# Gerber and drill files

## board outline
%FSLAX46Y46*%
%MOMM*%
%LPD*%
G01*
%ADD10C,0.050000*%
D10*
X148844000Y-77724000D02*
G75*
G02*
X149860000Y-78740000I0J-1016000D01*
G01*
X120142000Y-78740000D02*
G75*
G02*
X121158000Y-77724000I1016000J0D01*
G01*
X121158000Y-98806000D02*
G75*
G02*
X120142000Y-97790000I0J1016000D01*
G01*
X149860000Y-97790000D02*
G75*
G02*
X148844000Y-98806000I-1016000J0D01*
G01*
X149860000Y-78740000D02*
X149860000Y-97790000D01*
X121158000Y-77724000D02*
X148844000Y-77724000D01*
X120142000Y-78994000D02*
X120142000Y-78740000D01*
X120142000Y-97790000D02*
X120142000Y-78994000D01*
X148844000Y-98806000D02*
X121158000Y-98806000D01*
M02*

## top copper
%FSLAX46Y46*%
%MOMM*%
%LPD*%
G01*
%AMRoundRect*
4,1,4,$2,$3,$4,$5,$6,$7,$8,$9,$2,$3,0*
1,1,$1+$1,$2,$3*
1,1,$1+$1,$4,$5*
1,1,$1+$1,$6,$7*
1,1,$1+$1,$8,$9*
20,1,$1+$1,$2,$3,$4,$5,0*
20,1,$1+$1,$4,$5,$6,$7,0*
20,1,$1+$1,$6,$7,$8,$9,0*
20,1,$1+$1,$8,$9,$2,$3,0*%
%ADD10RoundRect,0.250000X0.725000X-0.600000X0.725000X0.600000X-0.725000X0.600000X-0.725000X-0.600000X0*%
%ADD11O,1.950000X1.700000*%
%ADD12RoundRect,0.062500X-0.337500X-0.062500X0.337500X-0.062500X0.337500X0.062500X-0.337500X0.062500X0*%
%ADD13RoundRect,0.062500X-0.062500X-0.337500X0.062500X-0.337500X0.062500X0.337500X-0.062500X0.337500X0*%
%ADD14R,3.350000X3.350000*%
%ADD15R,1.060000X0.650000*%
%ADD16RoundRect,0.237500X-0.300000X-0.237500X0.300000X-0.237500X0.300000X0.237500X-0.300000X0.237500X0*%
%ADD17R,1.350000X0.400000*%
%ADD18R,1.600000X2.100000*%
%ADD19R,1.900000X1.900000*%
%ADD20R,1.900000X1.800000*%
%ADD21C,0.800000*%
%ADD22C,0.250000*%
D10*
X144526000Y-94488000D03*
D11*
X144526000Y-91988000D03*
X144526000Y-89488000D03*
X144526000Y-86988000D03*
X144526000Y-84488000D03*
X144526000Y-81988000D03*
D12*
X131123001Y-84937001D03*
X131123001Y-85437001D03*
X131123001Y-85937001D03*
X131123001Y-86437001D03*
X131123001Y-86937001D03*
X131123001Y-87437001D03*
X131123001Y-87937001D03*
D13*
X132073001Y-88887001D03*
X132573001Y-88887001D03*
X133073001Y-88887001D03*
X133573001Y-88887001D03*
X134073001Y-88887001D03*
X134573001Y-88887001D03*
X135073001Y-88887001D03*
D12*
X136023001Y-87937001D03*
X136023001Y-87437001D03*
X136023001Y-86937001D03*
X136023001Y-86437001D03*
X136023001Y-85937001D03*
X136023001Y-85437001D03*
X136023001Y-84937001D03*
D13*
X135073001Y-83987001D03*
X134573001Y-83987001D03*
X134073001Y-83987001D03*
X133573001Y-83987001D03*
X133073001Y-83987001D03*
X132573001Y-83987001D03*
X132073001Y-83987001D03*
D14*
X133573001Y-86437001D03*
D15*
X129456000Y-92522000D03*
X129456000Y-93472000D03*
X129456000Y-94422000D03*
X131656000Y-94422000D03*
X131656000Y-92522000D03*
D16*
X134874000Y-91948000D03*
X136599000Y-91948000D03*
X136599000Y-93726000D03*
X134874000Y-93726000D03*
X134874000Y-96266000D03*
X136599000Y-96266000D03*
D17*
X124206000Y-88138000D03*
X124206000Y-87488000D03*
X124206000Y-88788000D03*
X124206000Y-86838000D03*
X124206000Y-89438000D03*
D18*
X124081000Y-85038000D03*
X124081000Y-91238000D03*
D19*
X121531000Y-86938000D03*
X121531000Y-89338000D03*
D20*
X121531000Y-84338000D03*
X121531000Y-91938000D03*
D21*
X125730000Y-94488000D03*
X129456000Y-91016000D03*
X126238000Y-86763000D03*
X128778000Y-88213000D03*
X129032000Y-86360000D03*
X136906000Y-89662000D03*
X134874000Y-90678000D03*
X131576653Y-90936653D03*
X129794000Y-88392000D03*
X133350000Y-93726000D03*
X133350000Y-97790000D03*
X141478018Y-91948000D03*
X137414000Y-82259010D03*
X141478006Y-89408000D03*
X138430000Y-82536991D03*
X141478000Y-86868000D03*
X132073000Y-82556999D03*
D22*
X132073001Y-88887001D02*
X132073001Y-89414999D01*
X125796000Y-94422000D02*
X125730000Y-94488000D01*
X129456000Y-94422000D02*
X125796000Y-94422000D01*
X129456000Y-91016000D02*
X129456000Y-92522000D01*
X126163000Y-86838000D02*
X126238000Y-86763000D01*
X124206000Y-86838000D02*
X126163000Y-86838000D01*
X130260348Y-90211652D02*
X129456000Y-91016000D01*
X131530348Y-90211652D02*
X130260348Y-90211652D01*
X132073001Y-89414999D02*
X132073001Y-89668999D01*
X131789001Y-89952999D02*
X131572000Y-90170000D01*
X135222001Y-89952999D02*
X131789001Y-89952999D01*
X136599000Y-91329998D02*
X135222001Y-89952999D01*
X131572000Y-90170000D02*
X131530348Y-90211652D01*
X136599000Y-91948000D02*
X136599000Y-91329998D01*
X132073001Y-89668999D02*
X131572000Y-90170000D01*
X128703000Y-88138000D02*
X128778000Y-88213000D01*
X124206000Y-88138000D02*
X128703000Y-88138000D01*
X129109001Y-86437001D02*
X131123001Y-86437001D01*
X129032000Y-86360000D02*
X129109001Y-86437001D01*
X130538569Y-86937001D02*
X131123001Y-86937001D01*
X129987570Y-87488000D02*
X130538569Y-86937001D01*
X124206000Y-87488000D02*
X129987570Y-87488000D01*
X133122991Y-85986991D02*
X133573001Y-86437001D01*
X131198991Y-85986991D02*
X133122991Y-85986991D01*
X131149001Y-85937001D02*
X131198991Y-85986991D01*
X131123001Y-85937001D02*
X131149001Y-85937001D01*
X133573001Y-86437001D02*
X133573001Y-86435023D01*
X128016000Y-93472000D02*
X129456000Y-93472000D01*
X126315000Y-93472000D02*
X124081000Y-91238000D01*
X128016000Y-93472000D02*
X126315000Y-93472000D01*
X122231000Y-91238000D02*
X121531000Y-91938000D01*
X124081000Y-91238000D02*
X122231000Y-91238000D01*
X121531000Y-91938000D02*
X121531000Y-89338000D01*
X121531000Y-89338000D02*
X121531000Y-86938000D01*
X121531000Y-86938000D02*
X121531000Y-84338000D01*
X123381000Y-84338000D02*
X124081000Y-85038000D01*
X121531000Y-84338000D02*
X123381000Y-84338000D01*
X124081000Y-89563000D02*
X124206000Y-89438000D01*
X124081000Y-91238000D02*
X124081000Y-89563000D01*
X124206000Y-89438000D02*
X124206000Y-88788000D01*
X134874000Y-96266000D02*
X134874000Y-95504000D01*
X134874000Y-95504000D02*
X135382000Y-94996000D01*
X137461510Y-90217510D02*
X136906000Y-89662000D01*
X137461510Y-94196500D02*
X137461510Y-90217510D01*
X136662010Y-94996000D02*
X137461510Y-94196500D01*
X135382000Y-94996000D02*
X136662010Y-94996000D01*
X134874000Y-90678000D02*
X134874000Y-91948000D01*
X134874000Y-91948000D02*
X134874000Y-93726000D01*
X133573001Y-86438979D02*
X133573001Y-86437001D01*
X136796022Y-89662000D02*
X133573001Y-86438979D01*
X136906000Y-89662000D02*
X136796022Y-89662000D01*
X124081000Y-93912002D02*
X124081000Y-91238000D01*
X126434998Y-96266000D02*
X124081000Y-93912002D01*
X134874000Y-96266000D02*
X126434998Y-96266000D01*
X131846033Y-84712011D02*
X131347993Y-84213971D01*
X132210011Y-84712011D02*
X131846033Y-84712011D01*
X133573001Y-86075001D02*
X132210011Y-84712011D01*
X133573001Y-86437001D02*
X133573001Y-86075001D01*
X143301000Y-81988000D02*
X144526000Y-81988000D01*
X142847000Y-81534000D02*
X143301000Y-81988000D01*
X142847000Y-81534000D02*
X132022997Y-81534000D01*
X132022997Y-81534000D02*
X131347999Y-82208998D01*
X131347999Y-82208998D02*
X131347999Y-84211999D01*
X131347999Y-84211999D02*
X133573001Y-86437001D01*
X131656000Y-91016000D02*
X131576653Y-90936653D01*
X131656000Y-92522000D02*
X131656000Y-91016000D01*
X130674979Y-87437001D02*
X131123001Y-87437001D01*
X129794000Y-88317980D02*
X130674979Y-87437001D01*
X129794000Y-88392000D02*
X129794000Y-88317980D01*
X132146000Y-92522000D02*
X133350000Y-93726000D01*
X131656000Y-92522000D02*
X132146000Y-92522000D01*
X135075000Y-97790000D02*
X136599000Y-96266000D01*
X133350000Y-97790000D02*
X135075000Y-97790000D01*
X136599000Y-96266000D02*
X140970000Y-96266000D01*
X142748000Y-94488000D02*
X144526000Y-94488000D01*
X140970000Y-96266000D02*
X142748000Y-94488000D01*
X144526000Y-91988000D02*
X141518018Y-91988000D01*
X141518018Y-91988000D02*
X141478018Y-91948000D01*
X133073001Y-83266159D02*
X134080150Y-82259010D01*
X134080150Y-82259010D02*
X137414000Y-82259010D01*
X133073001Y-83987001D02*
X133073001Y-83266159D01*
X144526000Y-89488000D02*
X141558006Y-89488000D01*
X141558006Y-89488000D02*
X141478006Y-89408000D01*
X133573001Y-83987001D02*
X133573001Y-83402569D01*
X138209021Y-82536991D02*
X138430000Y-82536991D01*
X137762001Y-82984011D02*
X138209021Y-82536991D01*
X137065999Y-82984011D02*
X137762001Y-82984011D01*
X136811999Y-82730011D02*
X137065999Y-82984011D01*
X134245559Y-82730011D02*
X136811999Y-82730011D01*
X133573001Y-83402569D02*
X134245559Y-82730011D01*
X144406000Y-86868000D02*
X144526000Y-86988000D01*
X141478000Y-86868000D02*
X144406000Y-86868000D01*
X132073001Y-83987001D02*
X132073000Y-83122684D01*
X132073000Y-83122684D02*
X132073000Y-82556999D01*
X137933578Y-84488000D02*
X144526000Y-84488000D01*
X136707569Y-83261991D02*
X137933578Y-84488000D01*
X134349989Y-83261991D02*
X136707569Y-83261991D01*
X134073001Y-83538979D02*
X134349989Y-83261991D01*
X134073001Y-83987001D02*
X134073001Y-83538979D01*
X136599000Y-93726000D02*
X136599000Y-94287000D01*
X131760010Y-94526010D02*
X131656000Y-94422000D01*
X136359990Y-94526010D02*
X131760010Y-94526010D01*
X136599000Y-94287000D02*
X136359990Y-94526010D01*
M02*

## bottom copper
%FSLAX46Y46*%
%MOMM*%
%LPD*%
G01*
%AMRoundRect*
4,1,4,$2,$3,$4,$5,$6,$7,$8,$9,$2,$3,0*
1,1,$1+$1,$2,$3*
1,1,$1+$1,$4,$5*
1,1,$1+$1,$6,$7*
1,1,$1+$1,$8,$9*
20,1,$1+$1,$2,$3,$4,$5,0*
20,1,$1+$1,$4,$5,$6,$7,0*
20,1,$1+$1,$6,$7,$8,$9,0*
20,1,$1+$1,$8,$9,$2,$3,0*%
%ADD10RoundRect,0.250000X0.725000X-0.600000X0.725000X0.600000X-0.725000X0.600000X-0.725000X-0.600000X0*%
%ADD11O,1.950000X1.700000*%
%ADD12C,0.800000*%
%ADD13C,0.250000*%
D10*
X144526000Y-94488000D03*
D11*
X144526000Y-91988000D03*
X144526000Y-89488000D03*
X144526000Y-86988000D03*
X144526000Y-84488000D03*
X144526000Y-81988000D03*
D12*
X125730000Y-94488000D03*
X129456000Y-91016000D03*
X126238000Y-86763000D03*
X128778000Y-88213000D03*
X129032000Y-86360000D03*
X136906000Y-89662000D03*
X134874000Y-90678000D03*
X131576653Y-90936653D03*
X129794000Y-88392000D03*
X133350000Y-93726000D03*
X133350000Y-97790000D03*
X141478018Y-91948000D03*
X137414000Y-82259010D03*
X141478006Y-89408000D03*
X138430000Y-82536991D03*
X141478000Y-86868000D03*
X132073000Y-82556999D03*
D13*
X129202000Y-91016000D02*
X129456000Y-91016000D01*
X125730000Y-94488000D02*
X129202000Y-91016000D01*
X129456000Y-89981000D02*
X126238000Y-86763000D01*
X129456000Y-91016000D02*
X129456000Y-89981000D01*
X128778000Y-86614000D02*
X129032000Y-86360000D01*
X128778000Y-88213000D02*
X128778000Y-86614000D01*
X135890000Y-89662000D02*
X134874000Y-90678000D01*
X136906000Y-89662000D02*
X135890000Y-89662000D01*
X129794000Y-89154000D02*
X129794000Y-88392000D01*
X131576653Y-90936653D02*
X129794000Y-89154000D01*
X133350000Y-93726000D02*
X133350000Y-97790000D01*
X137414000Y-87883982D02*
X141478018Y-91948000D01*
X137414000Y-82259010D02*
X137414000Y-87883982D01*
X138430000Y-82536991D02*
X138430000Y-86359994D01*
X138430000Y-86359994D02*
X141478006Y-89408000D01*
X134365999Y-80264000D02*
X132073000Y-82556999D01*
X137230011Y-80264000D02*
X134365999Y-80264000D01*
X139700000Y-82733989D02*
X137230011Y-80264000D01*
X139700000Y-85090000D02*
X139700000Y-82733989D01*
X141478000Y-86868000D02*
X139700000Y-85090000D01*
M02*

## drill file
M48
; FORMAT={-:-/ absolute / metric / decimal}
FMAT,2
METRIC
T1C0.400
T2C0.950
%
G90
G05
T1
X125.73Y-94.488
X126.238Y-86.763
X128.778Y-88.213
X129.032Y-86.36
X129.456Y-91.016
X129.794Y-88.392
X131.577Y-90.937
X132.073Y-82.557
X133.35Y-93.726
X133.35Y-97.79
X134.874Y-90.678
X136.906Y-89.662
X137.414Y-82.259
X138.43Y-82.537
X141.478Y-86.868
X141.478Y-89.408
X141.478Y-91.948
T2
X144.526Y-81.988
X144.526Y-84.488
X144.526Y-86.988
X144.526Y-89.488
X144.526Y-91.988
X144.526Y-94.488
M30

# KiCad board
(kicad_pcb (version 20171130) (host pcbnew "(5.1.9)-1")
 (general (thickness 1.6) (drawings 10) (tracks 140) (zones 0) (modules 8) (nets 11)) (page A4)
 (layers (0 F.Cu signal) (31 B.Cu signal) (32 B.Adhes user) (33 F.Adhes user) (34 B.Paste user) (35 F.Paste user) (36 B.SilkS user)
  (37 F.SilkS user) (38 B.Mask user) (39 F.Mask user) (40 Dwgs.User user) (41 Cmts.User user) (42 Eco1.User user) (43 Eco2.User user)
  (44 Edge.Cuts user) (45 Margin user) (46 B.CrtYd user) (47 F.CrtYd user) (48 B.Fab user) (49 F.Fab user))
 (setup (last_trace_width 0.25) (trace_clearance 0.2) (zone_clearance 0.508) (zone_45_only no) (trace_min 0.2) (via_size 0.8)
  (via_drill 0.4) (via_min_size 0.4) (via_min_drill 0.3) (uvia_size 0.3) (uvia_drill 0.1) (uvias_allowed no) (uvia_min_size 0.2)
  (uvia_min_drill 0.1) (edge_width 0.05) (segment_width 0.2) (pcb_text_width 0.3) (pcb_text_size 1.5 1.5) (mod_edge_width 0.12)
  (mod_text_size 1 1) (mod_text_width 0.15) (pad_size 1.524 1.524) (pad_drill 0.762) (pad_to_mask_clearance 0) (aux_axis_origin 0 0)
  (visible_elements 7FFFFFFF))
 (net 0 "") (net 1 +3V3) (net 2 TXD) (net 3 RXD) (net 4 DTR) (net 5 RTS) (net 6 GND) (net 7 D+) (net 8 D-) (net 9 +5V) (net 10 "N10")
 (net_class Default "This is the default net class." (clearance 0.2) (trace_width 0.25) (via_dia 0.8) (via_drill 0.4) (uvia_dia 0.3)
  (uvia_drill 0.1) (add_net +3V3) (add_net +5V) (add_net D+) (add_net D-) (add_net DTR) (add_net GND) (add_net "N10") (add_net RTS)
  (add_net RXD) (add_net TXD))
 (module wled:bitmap (layer F.Cu) (at 122.936 96.012)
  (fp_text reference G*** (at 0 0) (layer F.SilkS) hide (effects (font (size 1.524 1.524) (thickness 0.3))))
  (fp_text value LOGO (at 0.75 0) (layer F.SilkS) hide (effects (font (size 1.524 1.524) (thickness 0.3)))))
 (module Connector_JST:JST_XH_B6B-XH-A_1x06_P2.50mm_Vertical (layer F.Cu) (at 144.526 94.488 90)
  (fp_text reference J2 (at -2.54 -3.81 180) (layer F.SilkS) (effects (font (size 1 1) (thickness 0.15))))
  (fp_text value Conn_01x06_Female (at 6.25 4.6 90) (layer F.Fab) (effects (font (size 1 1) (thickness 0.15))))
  (pad 1 thru_hole roundrect (at 0 0 90) (size 1.7 1.95) (drill 0.95) (layers *.Cu *.Mask) (roundrect_rratio 0.1470588235294118)
   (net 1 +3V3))
  (pad 2 thru_hole oval (at 2.5 0 90) (size 1.7 1.95) (drill 0.95) (layers *.Cu *.Mask) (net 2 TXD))
  (pad 3 thru_hole oval (at 5 0 90) (size 1.7 1.95) (drill 0.95) (layers *.Cu *.Mask) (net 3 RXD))
  (pad 4 thru_hole oval (at 7.5 0 90) (size 1.7 1.95) (drill 0.95) (layers *.Cu *.Mask) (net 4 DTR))
  (pad 5 thru_hole oval (at 10 0 90) (size 1.7 1.95) (drill 0.95) (layers *.Cu *.Mask) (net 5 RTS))
  (pad 6 thru_hole oval (at 12.5 0 90) (size 1.7 1.95) (drill 0.95) (layers *.Cu *.Mask) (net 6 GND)))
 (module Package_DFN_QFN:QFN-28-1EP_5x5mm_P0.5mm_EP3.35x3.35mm (layer F.Cu) (at 133.573001 86.437001)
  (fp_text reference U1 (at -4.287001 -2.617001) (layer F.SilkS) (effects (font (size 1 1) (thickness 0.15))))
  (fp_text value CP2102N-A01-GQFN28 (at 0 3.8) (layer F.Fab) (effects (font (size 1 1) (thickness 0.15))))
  (pad 1 smd roundrect (at -2.45 -1.5) (size 0.8 0.25) (layers F.Cu F.Paste F.Mask) (roundrect_rratio 0.25))
  (pad 2 smd roundrect (at -2.45 -1) (size 0.8 0.25) (layers F.Cu F.Paste F.Mask) (roundrect_rratio 0.25))
  (pad 3 smd roundrect (at -2.45 -0.5) (size 0.8 0.25) (layers F.Cu F.Paste F.Mask) (roundrect_rratio 0.25) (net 6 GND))
  (pad 4 smd roundrect (at -2.45 0) (size 0.8 0.25) (layers F.Cu F.Paste F.Mask) (roundrect_rratio 0.25) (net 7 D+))
  (pad 5 smd roundrect (at -2.45 0.5) (size 0.8 0.25) (layers F.Cu F.Paste F.Mask) (roundrect_rratio 0.25) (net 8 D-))
  (pad 6 smd roundrect (at -2.45 1) (size 0.8 0.25) (layers F.Cu F.Paste F.Mask) (roundrect_rratio 0.25) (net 1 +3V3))
  (pad 7 smd roundrect (at -2.45 1.5) (size 0.8 0.25) (layers F.Cu F.Paste F.Mask) (roundrect_rratio 0.25))
  (pad 8 smd roundrect (at -1.5 2.45) (size 0.25 0.8) (layers F.Cu F.Paste F.Mask) (roundrect_rratio 0.25) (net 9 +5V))
  (pad 9 smd roundrect (at -1 2.45) (size 0.25 0.8) (layers F.Cu F.Paste F.Mask) (roundrect_rratio 0.25))
  (pad 10 smd roundrect (at -0.5 2.45) (size 0.25 0.8) (layers F.Cu F.Paste F.Mask) (roundrect_rratio 0.25))
  (pad 11 smd roundrect (at 0 2.45) (size 0.25 0.8) (layers F.Cu F.Paste F.Mask) (roundrect_rratio 0.25))
  (pad 12 smd roundrect (at 0.5 2.45) (size 0.25 0.8) (layers F.Cu F.Paste F.Mask) (roundrect_rratio 0.25))
  (pad 13 smd roundrect (at 1 2.45) (size 0.25 0.8) (layers F.Cu F.Paste F.Mask) (roundrect_rratio 0.25))
  (pad 14 smd roundrect (at 1.5 2.45) (size 0.25 0.8) (layers F.Cu F.Paste F.Mask) (roundrect_rratio 0.25))
  (pad 15 smd roundrect (at 2.45 1.5) (size 0.8 0.25) (layers F.Cu F.Paste F.Mask) (roundrect_rratio 0.25))
  (pad 16 smd roundrect (at 2.45 1) (size 0.8 0.25) (layers F.Cu F.Paste F.Mask) (roundrect_rratio 0.25))
  (pad 17 smd roundrect (at 2.45 0.5) (size 0.8 0.25) (layers F.Cu F.Paste F.Mask) (roundrect_rratio 0.25))
  (pad 18 smd roundrect (at 2.45 0) (size 0.8 0.25) (layers F.Cu F.Paste F.Mask) (roundrect_rratio 0.25))
  (pad 19 smd roundrect (at 2.45 -0.5) (size 0.8 0.25) (layers F.Cu F.Paste F.Mask) (roundrect_rratio 0.25))
  (pad 20 smd roundrect (at 2.45 -1) (size 0.8 0.25) (layers F.Cu F.Paste F.Mask) (roundrect_rratio 0.25))
  (pad 21 smd roundrect (at 2.45 -1.5) (size 0.8 0.25) (layers F.Cu F.Paste F.Mask) (roundrect_rratio 0.25))
  (pad 22 smd roundrect (at 1.5 -2.45) (size 0.25 0.8) (layers F.Cu F.Paste F.Mask) (roundrect_rratio 0.25))
  (pad 23 smd roundrect (at 1 -2.45) (size 0.25 0.8) (layers F.Cu F.Paste F.Mask) (roundrect_rratio 0.25))
  (pad 24 smd roundrect (at 0.5 -2.45) (size 0.25 0.8) (layers F.Cu F.Paste F.Mask) (roundrect_rratio 0.25) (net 5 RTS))
  (pad 25 smd roundrect (at 0 -2.45) (size 0.25 0.8) (layers F.Cu F.Paste F.Mask) (roundrect_rratio 0.25) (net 3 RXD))
  (pad 26 smd roundrect (at -0.5 -2.45) (size 0.25 0.8) (layers F.Cu F.Paste F.Mask) (roundrect_rratio 0.25) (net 2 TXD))
  (pad 27 smd roundrect (at -1 -2.45) (size 0.25 0.8) (layers F.Cu F.Paste F.Mask) (roundrect_rratio 0.25))
  (pad 28 smd roundrect (at -1.5 -2.45) (size 0.25 0.8) (layers F.Cu F.Paste F.Mask) (roundrect_rratio 0.25) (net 4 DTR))
  (pad 29 smd rect (at 0 0) (size 3.35 3.35) (layers F.Cu F.Mask) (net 6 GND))
  (pad "" smd roundrect (at -1.12 -1.12) (size 0.9 0.9) (layers F.Paste) (roundrect_rratio 0.25))
  (pad "" smd roundrect (at -1.12 0) (size 0.9 0.9) (layers F.Paste) (roundrect_rratio 0.25))
  (pad "" smd roundrect (at -1.12 1.12) (size 0.9 0.9) (layers F.Paste) (roundrect_rratio 0.25))
  (pad "" smd roundrect (at 0 -1.12) (size 0.9 0.9) (layers F.Paste) (roundrect_rratio 0.25))
  (pad "" smd roundrect (at 0 0) (size 0.9 0.9) (layers F.Paste) (roundrect_rratio 0.25))
  (pad "" smd roundrect (at 0 1.12) (size 0.9 0.9) (layers F.Paste) (roundrect_rratio 0.25))
  (pad "" smd roundrect (at 1.12 -1.12) (size 0.9 0.9) (layers F.Paste) (roundrect_rratio 0.25))
  (pad "" smd roundrect (at 1.12 0) (size 0.9 0.9) (layers F.Paste) (roundrect_rratio 0.25))
  (pad "" smd roundrect (at 1.12 1.12) (size 0.9 0.9) (layers F.Paste) (roundrect_rratio 0.25)))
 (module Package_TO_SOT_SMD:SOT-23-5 (layer F.Cu) (at 130.556 93.472)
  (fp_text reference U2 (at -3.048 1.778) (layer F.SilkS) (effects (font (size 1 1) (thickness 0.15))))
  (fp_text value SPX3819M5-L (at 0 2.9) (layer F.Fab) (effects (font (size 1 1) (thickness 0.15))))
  (pad 1 smd rect (at -1.1 -0.95) (size 1.06 0.65) (layers F.Cu F.Paste F.Mask) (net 9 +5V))
  (pad 2 smd rect (at -1.1 0) (size 1.06 0.65) (layers F.Cu F.Paste F.Mask) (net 6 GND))
  (pad 3 smd rect (at -1.1 0.95) (size 1.06 0.65) (layers F.Cu F.Paste F.Mask) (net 9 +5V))
  (pad 4 smd rect (at 1.1 0.95) (size 1.06 0.65) (layers F.Cu F.Paste F.Mask) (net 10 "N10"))
  (pad 5 smd rect (at 1.1 -0.95) (size 1.06 0.65) (layers F.Cu F.Paste F.Mask) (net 1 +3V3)))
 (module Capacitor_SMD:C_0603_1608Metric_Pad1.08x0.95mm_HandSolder (layer F.Cu) (at 135.7365 91.948)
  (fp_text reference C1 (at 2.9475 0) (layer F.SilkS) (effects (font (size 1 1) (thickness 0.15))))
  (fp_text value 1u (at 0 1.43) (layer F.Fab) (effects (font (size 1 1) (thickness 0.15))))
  (pad 1 smd roundrect (at -0.8625 0) (size 1.075 0.95) (layers F.Cu F.Paste F.Mask) (roundrect_rratio 0.25) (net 6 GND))
  (pad 2 smd roundrect (at 0.8625 0) (size 1.075 0.95) (layers F.Cu F.Paste F.Mask) (roundrect_rratio 0.25) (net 9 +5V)))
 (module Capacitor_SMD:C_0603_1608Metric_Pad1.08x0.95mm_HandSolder (layer F.Cu) (at 135.7365 93.726)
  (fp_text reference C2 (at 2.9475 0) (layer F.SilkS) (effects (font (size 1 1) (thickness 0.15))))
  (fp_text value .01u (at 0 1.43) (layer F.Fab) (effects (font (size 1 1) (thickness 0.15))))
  (pad 2 smd roundrect (at 0.8625 0) (size 1.075 0.95) (layers F.Cu F.Paste F.Mask) (roundrect_rratio 0.25) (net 10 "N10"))
  (pad 1 smd roundrect (at -0.8625 0) (size 1.075 0.95) (layers F.Cu F.Paste F.Mask) (roundrect_rratio 0.25) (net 6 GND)))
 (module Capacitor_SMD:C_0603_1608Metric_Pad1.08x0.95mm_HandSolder (layer F.Cu) (at 135.7365 96.266)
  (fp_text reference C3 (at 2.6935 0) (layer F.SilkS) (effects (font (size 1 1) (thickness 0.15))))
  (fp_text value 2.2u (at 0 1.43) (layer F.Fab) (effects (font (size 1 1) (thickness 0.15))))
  (pad 1 smd roundrect (at -0.8625 0) (size 1.075 0.95) (layers F.Cu F.Paste F.Mask) (roundrect_rratio 0.25) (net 6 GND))
  (pad 2 smd roundrect (at 0.8625 0) (size 1.075 0.95) (layers F.Cu F.Paste F.Mask) (roundrect_rratio 0.25) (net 1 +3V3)))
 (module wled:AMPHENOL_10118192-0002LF (layer F.Cu) (at 124.206 88.138 270)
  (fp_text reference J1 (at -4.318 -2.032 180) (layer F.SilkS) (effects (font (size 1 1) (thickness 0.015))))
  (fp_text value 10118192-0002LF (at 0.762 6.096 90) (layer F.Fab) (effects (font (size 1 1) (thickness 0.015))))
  (pad 3 smd rect (at 0 0 270) (size 0.4 1.35) (layers F.Cu F.Paste F.Mask) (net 7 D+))
  (pad 2 smd rect (at -0.65 0 270) (size 0.4 1.35) (layers F.Cu F.Paste F.Mask) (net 8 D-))
  (pad 4 smd rect (at 0.65 0 270) (size 0.4 1.35) (layers F.Cu F.Paste F.Mask) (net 6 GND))
  (pad 1 smd rect (at -1.3 0 270) (size 0.4 1.35) (layers F.Cu F.Paste F.Mask) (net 9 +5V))
  (pad 5 smd rect (at 1.3 0 270) (size 0.4 1.35) (layers F.Cu F.Paste F.Mask) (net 6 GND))
  (pad S1 smd rect (at -3.1 0.125 270) (size 2.1 1.6) (layers F.Cu F.Paste F.Mask) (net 6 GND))
  (pad S2 smd rect (at 3.1 0.125 270) (size 2.1 1.6) (layers F.Cu F.Paste F.Mask) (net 6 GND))
  (pad S4 smd rect (at -1.2 2.675 270) (size 1.9 1.9) (layers F.Cu F.Paste F.Mask) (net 6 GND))
  (pad S5 smd rect (at 1.2 2.675 270) (size 1.9 1.9) (layers F.Cu F.Paste F.Mask) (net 6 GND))
  (pad S3 smd rect (at -3.8 2.675 270) (size 1.8 1.9) (layers F.Cu F.Paste F.Mask) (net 6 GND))
  (pad S6 smd rect (at 3.8 2.675 270) (size 1.8 1.9) (layers F.Cu F.Paste F.Mask) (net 6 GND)))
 (gr_arc (start 148.844 78.74) (end 149.86 78.74) (angle -90) (layer Edge.Cuts) (width 0.05))
 (gr_arc (start 121.158 78.74) (end 121.158 77.724) (angle -90) (layer Edge.Cuts) (width 0.05))
 (gr_arc (start 121.158 97.79) (end 120.142 97.79) (angle -90) (layer Edge.Cuts) (width 0.05))
 (gr_arc (start 148.844 97.79) (end 148.844 98.806) (angle -90) (layer Edge.Cuts) (width 0.05))
 (gr_line (start 149.86 78.74) (end 149.86 97.79) (layer Edge.Cuts) (width 0.05))
 (gr_line (start 121.158 77.724) (end 148.844 77.724) (layer Edge.Cuts) (width 0.05))
 (gr_line (start 120.142 78.994) (end 120.142 78.74) (layer Edge.Cuts) (width 0.05))
 (gr_line (start 120.142 97.79) (end 120.142 78.994) (layer Edge.Cuts) (width 0.05))
 (gr_line (start 148.844 98.806) (end 121.158 98.806) (layer Edge.Cuts) (width 0.05))
 (segment (start 132.073001 88.887001) (end 132.073001 89.414999) (width 0.25) (layer F.Cu) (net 9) (status 10))
 (via (at 125.73 94.488) (size 0.8) (drill 0.4) (layers F.Cu B.Cu) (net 9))
 (segment (start 125.796 94.422) (end 125.73 94.488) (width 0.25) (layer F.Cu) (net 9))
 (segment (start 129.456 94.422) (end 125.796 94.422) (width 0.25) (layer F.Cu) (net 9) (status 10))
 (via (at 129.456 91.016) (size 0.8) (drill 0.4) (layers F.Cu B.Cu) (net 9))
 (segment (start 129.202 91.016) (end 129.456 91.016) (width 0.25) (layer B.Cu) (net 9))
 (segment (start 125.73 94.488) (end 129.202 91.016) (width 0.25) (layer B.Cu) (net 9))
 (segment (start 129.456 91.016) (end 129.456 92.522) (width 0.25) (layer F.Cu) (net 9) (status 20))
 (via (at 126.238 86.763) (size 0.8) (drill 0.4) (layers F.Cu B.Cu) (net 9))
 (segment (start 129.456 89.981) (end 126.238 86.763) (width 0.25) (layer B.Cu) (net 9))
 (segment (start 129.456 91.016) (end 129.456 89.981) (width 0.25) (layer B.Cu) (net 9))
 (segment (start 126.163 86.838) (end 126.238 86.763) (width 0.25) (layer F.Cu) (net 9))
 (segment (start 124.206 86.838) (end 126.163 86.838) (width 0.25) (layer F.Cu) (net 9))
 (segment (start 130.260348 90.211652) (end 129.456 91.016) (width 0.25) (layer F.Cu) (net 9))
 (segment (start 131.530348 90.211652) (end 130.260348 90.211652) (width 0.25) (layer F.Cu) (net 9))
 (segment (start 132.073001 89.414999) (end 132.073001 89.668999) (width 0.25) (layer F.Cu) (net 9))
 (segment (start 131.789001 89.952999) (end 131.572 90.17) (width 0.25) (layer F.Cu) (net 9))
 (segment (start 135.222001 89.952999) (end 131.789001 89.952999) (width 0.25) (layer F.Cu) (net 9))
 (segment (start 136.599 91.329998) (end 135.222001 89.952999) (width 0.25) (layer F.Cu) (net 9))
 (segment (start 131.572 90.17) (end 131.530348 90.211652) (width 0.25) (layer F.Cu) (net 9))
 (segment (start 136.599 91.948) (end 136.599 91.329998) (width 0.25) (layer F.Cu) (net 9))
 (segment (start 132.073001 89.668999) (end 131.572 90.17) (width 0.25) (layer F.Cu) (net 9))
 (via (at 128.778 88.213) (size 0.8) (drill 0.4) (layers F.Cu B.Cu) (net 7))
 (segment (start 128.703 88.138) (end 128.778 88.213) (width 0.25) (layer F.Cu) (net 7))
 (segment (start 124.206 88.138) (end 128.703 88.138) (width 0.25) (layer F.Cu) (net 7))
 (via (at 129.032 86.36) (size 0.8) (drill 0.4) (layers F.Cu B.Cu) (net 7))
 (segment (start 128.778 86.614) (end 129.032 86.36) (width 0.25) (layer B.Cu) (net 7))
 (segment (start 128.778 88.213) (end 128.778 86.614) (width 0.25) (layer B.Cu) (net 7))
 (segment (start 129.109001 86.437001) (end 131.123001 86.437001) (width 0.25) (layer F.Cu) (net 7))
 (segment (start 129.032 86.36) (end 129.109001 86.437001) (width 0.25) (layer F.Cu) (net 7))
 (segment (start 130.538569 86.937001) (end 131.123001 86.937001) (width 0.25) (layer F.Cu) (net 8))
 (segment (start 129.98757 87.488) (end 130.538569 86.937001) (width 0.25) (layer F.Cu) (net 8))
 (segment (start 124.206 87.488) (end 129.98757 87.488) (width 0.25) (layer F.Cu) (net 8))
 (segment (start 133.122991 85.986991) (end 133.573001 86.437001) (width 0.25) (layer F.Cu) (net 6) (status 30))
 (segment (start 131.198991 85.986991) (end 133.122991 85.986991) (width 0.25) (layer F.Cu) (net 6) (status 30))
 (segment (start 131.149001 85.937001) (end 131.198991 85.986991) (width 0.25) (layer F.Cu) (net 6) (status 30))
 (segment (start 131.123001 85.937001) (end 131.149001 85.937001) (width 0.25) (layer F.Cu) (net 6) (status 30))
 (segment (start 133.573001 86.437001) (end 133.573001 86.435023) (width 0.25) (layer F.Cu) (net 6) (status 30))
 (segment (start 128.016 93.472) (end 129.456 93.472) (width 0.25) (layer F.Cu) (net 6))
 (segment (start 126.315 93.472) (end 124.081 91.238) (width 0.25) (layer F.Cu) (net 6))
 (segment (start 128.016 93.472) (end 126.315 93.472) (width 0.25) (layer F.Cu) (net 6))
 (segment (start 122.231 91.238) (end 121.531 91.938) (width 0.25) (layer F.Cu) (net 6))
 (segment (start 124.081 91.238) (end 122.231 91.238) (width 0.25) (layer F.Cu) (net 6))
 (segment (start 121.531 91.938) (end 121.531 89.338) (width 0.25) (layer F.Cu) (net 6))
 (segment (start 121.531 89.338) (end 121.531 86.938) (width 0.25) (layer F.Cu) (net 6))
 (segment (start 121.531 86.938) (end 121.531 84.338) (width 0.25) (layer F.Cu) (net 6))
 (segment (start 123.381 84.338) (end 124.081 85.038) (width 0.25) (layer F.Cu) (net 6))
 (segment (start 121.531 84.338) (end 123.381 84.338) (width 0.25) (layer F.Cu) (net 6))
 (segment (start 124.081 89.563) (end 124.206 89.438) (width 0.25) (layer F.Cu) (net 6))
 (segment (start 124.081 91.238) (end 124.081 89.563) (width 0.25) (layer F.Cu) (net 6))
 (segment (start 124.206 89.438) (end 124.206 88.788) (width 0.25) (layer F.Cu) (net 6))
 (segment (start 134.874 96.266) (end 134.874 95.504) (width 0.25) (layer F.Cu) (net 6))
 (segment (start 134.874 95.504) (end 135.382 94.996) (width 0.25) (layer F.Cu) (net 6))
 (via (at 136.906 89.662) (size 0.8) (drill 0.4) (layers F.Cu B.Cu) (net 6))
 (segment (start 137.46151 90.21751) (end 136.906 89.662) (width 0.25) (layer F.Cu) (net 6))
 (segment (start 137.46151 94.1965) (end 137.46151 90.21751) (width 0.25) (layer F.Cu) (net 6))
 (segment (start 136.66201 94.996) (end 137.46151 94.1965) (width 0.25) (layer F.Cu) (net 6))
 (segment (start 135.382 94.996) (end 136.66201 94.996) (width 0.25) (layer F.Cu) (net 6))
 (via (at 134.874 90.678) (size 0.8) (drill 0.4) (layers F.Cu B.Cu) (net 6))
 (segment (start 135.89 89.662) (end 134.874 90.678) (width 0.25) (layer B.Cu) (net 6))
 (segment (start 136.906 89.662) (end 135.89 89.662) (width 0.25) (layer B.Cu) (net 6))
 (segment (start 134.874 90.678) (end 134.874 91.948) (width 0.25) (layer F.Cu) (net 6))
 (segment (start 134.874 91.948) (end 134.874 93.726) (width 0.25) (layer F.Cu) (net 6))
 (segment (start 133.573001 86.438979) (end 133.573001 86.437001) (width 0.25) (layer F.Cu) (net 6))
 (segment (start 136.796022 89.662) (end 133.573001 86.438979) (width 0.25) (layer F.Cu) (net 6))
 (segment (start 136.906 89.662) (end 136.796022 89.662) (width 0.25) (layer F.Cu) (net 6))
 (segment (start 124.081 93.912002) (end 124.081 91.238) (width 0.25) (layer F.Cu) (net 6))
 (segment (start 126.434998 96.266) (end 124.081 93.912002) (width 0.25) (layer F.Cu) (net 6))
 (segment (start 134.874 96.266) (end 126.434998 96.266) (width 0.25) (layer F.Cu) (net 6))
 (segment (start 131.846033 84.712011) (end 131.347993 84.213971) (width 0.25) (layer F.Cu) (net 6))
 (segment (start 132.210011 84.712011) (end 131.846033 84.712011) (width 0.25) (layer F.Cu) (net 6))
 (segment (start 133.573001 86.075001) (end 132.210011 84.712011) (width 0.25) (layer F.Cu) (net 6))
 (segment (start 133.573001 86.437001) (end 133.573001 86.075001) (width 0.25) (layer F.Cu) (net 6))
 (segment (start 143.301 81.988) (end 144.526 81.988) (width 0.25) (layer F.Cu) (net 6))
 (segment (start 142.847 81.534) (end 143.301 81.988) (width 0.25) (layer F.Cu) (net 6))
 (segment (start 142.847 81.534) (end 132.022997 81.534) (width 0.25) (layer F.Cu) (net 6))
 (segment (start 132.022997 81.534) (end 131.347999 82.208998) (width 0.25) (layer F.Cu) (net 6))
 (segment (start 131.347999 82.208998) (end 131.347999 84.211999) (width 0.25) (layer F.Cu) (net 6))
 (segment (start 131.347999 84.211999) (end 133.573001 86.437001) (width 0.25) (layer F.Cu) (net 6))
 (via (at 131.576653 90.936653) (size 0.8) (drill 0.4) (layers F.Cu B.Cu) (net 1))
 (segment (start 131.656 91.016) (end 131.576653 90.936653) (width 0.25) (layer F.Cu) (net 1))
 (segment (start 131.656 92.522) (end 131.656 91.016) (width 0.25) (layer F.Cu) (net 1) (status 10))
 (via (at 129.794 88.392) (size 0.8) (drill 0.4) (layers F.Cu B.Cu) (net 1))
 (segment (start 129.794 89.154) (end 129.794 88.392) (width 0.25) (layer B.Cu) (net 1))
 (segment (start 131.576653 90.936653) (end 129.794 89.154) (width 0.25) (layer B.Cu) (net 1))
 (segment (start 130.674979 87.437001) (end 131.123001 87.437001) (width 0.25) (layer F.Cu) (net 1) (status 20))
 (segment (start 129.794 88.31798) (end 130.674979 87.437001) (width 0.25) (layer F.Cu) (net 1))
 (segment (start 129.794 88.392) (end 129.794 88.31798) (width 0.25) (layer F.Cu) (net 1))
 (via (at 133.35 93.726) (size 0.8) (drill 0.4) (layers F.Cu B.Cu) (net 1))
 (segment (start 132.146 92.522) (end 133.35 93.726) (width 0.25) (layer F.Cu) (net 1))
 (segment (start 131.656 92.522) (end 132.146 92.522) (width 0.25) (layer F.Cu) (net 1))
 (via (at 133.35 97.79) (size 0.8) (drill 0.4) (layers F.Cu B.Cu) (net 1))
 (segment (start 133.35 93.726) (end 133.35 97.79) (width 0.25) (layer B.Cu) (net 1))
 (segment (start 135.075 97.79) (end 136.599 96.266) (width 0.25) (layer F.Cu) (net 1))
 (segment (start 133.35 97.79) (end 135.075 97.79) (width 0.25) (layer F.Cu) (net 1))
 (segment (start 136.599 96.266) (end 140.97 96.266) (width 0.25) (layer F.Cu) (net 1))
 (segment (start 142.748 94.488) (end 144.526 94.488) (width 0.25) (layer F.Cu) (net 1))
 (segment (start 140.97 96.266) (end 142.748 94.488) (width 0.25) (layer F.Cu) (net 1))
 (via (at 141.478018 91.948) (size 0.8) (drill 0.4) (layers F.Cu B.Cu) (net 2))
 (segment (start 144.526 91.988) (end 141.518018 91.988) (width 0.25) (layer F.Cu) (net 2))
 (segment (start 141.518018 91.988) (end 141.478018 91.948) (width 0.25) (layer F.Cu) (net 2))
 (segment (start 133.073001 83.266159) (end 134.08015 82.25901) (width 0.25) (layer F.Cu) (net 2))
 (segment (start 134.08015 82.25901) (end 137.414 82.25901) (width 0.25) (layer F.Cu) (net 2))
 (via (at 137.414 82.25901) (size 0.8) (drill 0.4) (layers F.Cu B.Cu) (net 2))
 (segment (start 133.073001 83.987001) (end 133.073001 83.266159) (width 0.25) (layer F.Cu) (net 2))
 (segment (start 137.414 87.883982) (end 141.478018 91.948) (width 0.25) (layer B.Cu) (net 2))
 (segment (start 137.414 82.25901) (end 137.414 87.883982) (width 0.25) (layer B.Cu) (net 2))
 (via (at 141.478006 89.408) (size 0.8) (drill 0.4) (layers F.Cu B.Cu) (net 3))
 (segment (start 144.526 89.488) (end 141.558006 89.488) (width 0.25) (layer F.Cu) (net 3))
 (segment (start 141.558006 89.488) (end 141.478006 89.408) (width 0.25) (layer F.Cu) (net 3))
 (segment (start 138.43 82.536991) (end 138.43 86.359994) (width 0.25) (layer B.Cu) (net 3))
 (segment (start 133.573001 83.987001) (end 133.573001 83.402569) (width 0.25) (layer F.Cu) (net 3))
 (segment (start 138.209021 82.536991) (end 138.43 82.536991) (width 0.25) (layer F.Cu) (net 3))
 (segment (start 137.762001 82.984011) (end 138.209021 82.536991) (width 0.25) (layer F.Cu) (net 3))
 (segment (start 137.065999 82.984011) (end 137.762001 82.984011) (width 0.25) (layer F.Cu) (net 3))
 (segment (start 136.811999 82.730011) (end 137.065999 82.984011) (width 0.25) (layer F.Cu) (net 3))
 (via (at 138.43 82.536991) (size 0.8) (drill 0.4) (layers F.Cu B.Cu) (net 3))
 (segment (start 134.245559 82.730011) (end 136.811999 82.730011) (width 0.25) (layer F.Cu) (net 3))
 (segment (start 138.43 86.359994) (end 141.478006 89.408) (width 0.25) (layer B.Cu) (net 3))
 (segment (start 133.573001 83.402569) (end 134.245559 82.730011) (width 0.25) (layer F.Cu) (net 3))
 (via (at 141.478 86.868) (size 0.8) (drill 0.4) (layers F.Cu B.Cu) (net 4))
 (segment (start 144.406 86.868) (end 144.526 86.988) (width 0.25) (layer F.Cu) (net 4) (status 30))
 (segment (start 141.478 86.868) (end 144.406 86.868) (width 0.25) (layer F.Cu) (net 4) (status 20))
 (via (at 132.073 82.556999) (size 0.8) (drill 0.4) (layers F.Cu B.Cu) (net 4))
 (segment (start 132.073001 83.987001) (end 132.073 83.122684) (width 0.25) (layer F.Cu) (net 4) (status 10))
 (segment (start 132.073 83.122684) (end 132.073 82.556999) (width 0.25) (layer F.Cu) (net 4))
 (segment (start 134.365999 80.264) (end 132.073 82.556999) (width 0.25) (layer B.Cu) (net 4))
 (segment (start 137.230011 80.264) (end 134.365999 80.264) (width 0.25) (layer B.Cu) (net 4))
 (segment (start 139.7 82.733989) (end 137.230011 80.264) (width 0.25) (layer B.Cu) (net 4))
 (segment (start 139.7 85.09) (end 139.7 82.733989) (width 0.25) (layer B.Cu) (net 4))
 (segment (start 141.478 86.868) (end 139.7 85.09) (width 0.25) (layer B.Cu) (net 4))
 (segment (start 137.933578 84.488) (end 144.526 84.488) (width 0.25) (layer F.Cu) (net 5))
 (segment (start 136.707569 83.261991) (end 137.933578 84.488) (width 0.25) (layer F.Cu) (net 5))
 (segment (start 134.349989 83.261991) (end 136.707569 83.261991) (width 0.25) (layer F.Cu) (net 5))
 (segment (start 134.073001 83.538979) (end 134.349989 83.261991) (width 0.25) (layer F.Cu) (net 5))
 (segment (start 134.073001 83.987001) (end 134.073001 83.538979) (width 0.25) (layer F.Cu) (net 5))
 (segment (start 136.599 93.726) (end 136.599 94.287) (width 0.25) (layer F.Cu) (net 10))
 (segment (start 131.76001 94.52601) (end 131.656 94.422) (width 0.25) (layer F.Cu) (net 10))
 (segment (start 136.35999 94.52601) (end 131.76001 94.52601) (width 0.25) (layer F.Cu) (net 10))
 (segment (start 136.599 94.287) (end 136.35999 94.52601) (width 0.25) (layer F.Cu) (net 10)))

